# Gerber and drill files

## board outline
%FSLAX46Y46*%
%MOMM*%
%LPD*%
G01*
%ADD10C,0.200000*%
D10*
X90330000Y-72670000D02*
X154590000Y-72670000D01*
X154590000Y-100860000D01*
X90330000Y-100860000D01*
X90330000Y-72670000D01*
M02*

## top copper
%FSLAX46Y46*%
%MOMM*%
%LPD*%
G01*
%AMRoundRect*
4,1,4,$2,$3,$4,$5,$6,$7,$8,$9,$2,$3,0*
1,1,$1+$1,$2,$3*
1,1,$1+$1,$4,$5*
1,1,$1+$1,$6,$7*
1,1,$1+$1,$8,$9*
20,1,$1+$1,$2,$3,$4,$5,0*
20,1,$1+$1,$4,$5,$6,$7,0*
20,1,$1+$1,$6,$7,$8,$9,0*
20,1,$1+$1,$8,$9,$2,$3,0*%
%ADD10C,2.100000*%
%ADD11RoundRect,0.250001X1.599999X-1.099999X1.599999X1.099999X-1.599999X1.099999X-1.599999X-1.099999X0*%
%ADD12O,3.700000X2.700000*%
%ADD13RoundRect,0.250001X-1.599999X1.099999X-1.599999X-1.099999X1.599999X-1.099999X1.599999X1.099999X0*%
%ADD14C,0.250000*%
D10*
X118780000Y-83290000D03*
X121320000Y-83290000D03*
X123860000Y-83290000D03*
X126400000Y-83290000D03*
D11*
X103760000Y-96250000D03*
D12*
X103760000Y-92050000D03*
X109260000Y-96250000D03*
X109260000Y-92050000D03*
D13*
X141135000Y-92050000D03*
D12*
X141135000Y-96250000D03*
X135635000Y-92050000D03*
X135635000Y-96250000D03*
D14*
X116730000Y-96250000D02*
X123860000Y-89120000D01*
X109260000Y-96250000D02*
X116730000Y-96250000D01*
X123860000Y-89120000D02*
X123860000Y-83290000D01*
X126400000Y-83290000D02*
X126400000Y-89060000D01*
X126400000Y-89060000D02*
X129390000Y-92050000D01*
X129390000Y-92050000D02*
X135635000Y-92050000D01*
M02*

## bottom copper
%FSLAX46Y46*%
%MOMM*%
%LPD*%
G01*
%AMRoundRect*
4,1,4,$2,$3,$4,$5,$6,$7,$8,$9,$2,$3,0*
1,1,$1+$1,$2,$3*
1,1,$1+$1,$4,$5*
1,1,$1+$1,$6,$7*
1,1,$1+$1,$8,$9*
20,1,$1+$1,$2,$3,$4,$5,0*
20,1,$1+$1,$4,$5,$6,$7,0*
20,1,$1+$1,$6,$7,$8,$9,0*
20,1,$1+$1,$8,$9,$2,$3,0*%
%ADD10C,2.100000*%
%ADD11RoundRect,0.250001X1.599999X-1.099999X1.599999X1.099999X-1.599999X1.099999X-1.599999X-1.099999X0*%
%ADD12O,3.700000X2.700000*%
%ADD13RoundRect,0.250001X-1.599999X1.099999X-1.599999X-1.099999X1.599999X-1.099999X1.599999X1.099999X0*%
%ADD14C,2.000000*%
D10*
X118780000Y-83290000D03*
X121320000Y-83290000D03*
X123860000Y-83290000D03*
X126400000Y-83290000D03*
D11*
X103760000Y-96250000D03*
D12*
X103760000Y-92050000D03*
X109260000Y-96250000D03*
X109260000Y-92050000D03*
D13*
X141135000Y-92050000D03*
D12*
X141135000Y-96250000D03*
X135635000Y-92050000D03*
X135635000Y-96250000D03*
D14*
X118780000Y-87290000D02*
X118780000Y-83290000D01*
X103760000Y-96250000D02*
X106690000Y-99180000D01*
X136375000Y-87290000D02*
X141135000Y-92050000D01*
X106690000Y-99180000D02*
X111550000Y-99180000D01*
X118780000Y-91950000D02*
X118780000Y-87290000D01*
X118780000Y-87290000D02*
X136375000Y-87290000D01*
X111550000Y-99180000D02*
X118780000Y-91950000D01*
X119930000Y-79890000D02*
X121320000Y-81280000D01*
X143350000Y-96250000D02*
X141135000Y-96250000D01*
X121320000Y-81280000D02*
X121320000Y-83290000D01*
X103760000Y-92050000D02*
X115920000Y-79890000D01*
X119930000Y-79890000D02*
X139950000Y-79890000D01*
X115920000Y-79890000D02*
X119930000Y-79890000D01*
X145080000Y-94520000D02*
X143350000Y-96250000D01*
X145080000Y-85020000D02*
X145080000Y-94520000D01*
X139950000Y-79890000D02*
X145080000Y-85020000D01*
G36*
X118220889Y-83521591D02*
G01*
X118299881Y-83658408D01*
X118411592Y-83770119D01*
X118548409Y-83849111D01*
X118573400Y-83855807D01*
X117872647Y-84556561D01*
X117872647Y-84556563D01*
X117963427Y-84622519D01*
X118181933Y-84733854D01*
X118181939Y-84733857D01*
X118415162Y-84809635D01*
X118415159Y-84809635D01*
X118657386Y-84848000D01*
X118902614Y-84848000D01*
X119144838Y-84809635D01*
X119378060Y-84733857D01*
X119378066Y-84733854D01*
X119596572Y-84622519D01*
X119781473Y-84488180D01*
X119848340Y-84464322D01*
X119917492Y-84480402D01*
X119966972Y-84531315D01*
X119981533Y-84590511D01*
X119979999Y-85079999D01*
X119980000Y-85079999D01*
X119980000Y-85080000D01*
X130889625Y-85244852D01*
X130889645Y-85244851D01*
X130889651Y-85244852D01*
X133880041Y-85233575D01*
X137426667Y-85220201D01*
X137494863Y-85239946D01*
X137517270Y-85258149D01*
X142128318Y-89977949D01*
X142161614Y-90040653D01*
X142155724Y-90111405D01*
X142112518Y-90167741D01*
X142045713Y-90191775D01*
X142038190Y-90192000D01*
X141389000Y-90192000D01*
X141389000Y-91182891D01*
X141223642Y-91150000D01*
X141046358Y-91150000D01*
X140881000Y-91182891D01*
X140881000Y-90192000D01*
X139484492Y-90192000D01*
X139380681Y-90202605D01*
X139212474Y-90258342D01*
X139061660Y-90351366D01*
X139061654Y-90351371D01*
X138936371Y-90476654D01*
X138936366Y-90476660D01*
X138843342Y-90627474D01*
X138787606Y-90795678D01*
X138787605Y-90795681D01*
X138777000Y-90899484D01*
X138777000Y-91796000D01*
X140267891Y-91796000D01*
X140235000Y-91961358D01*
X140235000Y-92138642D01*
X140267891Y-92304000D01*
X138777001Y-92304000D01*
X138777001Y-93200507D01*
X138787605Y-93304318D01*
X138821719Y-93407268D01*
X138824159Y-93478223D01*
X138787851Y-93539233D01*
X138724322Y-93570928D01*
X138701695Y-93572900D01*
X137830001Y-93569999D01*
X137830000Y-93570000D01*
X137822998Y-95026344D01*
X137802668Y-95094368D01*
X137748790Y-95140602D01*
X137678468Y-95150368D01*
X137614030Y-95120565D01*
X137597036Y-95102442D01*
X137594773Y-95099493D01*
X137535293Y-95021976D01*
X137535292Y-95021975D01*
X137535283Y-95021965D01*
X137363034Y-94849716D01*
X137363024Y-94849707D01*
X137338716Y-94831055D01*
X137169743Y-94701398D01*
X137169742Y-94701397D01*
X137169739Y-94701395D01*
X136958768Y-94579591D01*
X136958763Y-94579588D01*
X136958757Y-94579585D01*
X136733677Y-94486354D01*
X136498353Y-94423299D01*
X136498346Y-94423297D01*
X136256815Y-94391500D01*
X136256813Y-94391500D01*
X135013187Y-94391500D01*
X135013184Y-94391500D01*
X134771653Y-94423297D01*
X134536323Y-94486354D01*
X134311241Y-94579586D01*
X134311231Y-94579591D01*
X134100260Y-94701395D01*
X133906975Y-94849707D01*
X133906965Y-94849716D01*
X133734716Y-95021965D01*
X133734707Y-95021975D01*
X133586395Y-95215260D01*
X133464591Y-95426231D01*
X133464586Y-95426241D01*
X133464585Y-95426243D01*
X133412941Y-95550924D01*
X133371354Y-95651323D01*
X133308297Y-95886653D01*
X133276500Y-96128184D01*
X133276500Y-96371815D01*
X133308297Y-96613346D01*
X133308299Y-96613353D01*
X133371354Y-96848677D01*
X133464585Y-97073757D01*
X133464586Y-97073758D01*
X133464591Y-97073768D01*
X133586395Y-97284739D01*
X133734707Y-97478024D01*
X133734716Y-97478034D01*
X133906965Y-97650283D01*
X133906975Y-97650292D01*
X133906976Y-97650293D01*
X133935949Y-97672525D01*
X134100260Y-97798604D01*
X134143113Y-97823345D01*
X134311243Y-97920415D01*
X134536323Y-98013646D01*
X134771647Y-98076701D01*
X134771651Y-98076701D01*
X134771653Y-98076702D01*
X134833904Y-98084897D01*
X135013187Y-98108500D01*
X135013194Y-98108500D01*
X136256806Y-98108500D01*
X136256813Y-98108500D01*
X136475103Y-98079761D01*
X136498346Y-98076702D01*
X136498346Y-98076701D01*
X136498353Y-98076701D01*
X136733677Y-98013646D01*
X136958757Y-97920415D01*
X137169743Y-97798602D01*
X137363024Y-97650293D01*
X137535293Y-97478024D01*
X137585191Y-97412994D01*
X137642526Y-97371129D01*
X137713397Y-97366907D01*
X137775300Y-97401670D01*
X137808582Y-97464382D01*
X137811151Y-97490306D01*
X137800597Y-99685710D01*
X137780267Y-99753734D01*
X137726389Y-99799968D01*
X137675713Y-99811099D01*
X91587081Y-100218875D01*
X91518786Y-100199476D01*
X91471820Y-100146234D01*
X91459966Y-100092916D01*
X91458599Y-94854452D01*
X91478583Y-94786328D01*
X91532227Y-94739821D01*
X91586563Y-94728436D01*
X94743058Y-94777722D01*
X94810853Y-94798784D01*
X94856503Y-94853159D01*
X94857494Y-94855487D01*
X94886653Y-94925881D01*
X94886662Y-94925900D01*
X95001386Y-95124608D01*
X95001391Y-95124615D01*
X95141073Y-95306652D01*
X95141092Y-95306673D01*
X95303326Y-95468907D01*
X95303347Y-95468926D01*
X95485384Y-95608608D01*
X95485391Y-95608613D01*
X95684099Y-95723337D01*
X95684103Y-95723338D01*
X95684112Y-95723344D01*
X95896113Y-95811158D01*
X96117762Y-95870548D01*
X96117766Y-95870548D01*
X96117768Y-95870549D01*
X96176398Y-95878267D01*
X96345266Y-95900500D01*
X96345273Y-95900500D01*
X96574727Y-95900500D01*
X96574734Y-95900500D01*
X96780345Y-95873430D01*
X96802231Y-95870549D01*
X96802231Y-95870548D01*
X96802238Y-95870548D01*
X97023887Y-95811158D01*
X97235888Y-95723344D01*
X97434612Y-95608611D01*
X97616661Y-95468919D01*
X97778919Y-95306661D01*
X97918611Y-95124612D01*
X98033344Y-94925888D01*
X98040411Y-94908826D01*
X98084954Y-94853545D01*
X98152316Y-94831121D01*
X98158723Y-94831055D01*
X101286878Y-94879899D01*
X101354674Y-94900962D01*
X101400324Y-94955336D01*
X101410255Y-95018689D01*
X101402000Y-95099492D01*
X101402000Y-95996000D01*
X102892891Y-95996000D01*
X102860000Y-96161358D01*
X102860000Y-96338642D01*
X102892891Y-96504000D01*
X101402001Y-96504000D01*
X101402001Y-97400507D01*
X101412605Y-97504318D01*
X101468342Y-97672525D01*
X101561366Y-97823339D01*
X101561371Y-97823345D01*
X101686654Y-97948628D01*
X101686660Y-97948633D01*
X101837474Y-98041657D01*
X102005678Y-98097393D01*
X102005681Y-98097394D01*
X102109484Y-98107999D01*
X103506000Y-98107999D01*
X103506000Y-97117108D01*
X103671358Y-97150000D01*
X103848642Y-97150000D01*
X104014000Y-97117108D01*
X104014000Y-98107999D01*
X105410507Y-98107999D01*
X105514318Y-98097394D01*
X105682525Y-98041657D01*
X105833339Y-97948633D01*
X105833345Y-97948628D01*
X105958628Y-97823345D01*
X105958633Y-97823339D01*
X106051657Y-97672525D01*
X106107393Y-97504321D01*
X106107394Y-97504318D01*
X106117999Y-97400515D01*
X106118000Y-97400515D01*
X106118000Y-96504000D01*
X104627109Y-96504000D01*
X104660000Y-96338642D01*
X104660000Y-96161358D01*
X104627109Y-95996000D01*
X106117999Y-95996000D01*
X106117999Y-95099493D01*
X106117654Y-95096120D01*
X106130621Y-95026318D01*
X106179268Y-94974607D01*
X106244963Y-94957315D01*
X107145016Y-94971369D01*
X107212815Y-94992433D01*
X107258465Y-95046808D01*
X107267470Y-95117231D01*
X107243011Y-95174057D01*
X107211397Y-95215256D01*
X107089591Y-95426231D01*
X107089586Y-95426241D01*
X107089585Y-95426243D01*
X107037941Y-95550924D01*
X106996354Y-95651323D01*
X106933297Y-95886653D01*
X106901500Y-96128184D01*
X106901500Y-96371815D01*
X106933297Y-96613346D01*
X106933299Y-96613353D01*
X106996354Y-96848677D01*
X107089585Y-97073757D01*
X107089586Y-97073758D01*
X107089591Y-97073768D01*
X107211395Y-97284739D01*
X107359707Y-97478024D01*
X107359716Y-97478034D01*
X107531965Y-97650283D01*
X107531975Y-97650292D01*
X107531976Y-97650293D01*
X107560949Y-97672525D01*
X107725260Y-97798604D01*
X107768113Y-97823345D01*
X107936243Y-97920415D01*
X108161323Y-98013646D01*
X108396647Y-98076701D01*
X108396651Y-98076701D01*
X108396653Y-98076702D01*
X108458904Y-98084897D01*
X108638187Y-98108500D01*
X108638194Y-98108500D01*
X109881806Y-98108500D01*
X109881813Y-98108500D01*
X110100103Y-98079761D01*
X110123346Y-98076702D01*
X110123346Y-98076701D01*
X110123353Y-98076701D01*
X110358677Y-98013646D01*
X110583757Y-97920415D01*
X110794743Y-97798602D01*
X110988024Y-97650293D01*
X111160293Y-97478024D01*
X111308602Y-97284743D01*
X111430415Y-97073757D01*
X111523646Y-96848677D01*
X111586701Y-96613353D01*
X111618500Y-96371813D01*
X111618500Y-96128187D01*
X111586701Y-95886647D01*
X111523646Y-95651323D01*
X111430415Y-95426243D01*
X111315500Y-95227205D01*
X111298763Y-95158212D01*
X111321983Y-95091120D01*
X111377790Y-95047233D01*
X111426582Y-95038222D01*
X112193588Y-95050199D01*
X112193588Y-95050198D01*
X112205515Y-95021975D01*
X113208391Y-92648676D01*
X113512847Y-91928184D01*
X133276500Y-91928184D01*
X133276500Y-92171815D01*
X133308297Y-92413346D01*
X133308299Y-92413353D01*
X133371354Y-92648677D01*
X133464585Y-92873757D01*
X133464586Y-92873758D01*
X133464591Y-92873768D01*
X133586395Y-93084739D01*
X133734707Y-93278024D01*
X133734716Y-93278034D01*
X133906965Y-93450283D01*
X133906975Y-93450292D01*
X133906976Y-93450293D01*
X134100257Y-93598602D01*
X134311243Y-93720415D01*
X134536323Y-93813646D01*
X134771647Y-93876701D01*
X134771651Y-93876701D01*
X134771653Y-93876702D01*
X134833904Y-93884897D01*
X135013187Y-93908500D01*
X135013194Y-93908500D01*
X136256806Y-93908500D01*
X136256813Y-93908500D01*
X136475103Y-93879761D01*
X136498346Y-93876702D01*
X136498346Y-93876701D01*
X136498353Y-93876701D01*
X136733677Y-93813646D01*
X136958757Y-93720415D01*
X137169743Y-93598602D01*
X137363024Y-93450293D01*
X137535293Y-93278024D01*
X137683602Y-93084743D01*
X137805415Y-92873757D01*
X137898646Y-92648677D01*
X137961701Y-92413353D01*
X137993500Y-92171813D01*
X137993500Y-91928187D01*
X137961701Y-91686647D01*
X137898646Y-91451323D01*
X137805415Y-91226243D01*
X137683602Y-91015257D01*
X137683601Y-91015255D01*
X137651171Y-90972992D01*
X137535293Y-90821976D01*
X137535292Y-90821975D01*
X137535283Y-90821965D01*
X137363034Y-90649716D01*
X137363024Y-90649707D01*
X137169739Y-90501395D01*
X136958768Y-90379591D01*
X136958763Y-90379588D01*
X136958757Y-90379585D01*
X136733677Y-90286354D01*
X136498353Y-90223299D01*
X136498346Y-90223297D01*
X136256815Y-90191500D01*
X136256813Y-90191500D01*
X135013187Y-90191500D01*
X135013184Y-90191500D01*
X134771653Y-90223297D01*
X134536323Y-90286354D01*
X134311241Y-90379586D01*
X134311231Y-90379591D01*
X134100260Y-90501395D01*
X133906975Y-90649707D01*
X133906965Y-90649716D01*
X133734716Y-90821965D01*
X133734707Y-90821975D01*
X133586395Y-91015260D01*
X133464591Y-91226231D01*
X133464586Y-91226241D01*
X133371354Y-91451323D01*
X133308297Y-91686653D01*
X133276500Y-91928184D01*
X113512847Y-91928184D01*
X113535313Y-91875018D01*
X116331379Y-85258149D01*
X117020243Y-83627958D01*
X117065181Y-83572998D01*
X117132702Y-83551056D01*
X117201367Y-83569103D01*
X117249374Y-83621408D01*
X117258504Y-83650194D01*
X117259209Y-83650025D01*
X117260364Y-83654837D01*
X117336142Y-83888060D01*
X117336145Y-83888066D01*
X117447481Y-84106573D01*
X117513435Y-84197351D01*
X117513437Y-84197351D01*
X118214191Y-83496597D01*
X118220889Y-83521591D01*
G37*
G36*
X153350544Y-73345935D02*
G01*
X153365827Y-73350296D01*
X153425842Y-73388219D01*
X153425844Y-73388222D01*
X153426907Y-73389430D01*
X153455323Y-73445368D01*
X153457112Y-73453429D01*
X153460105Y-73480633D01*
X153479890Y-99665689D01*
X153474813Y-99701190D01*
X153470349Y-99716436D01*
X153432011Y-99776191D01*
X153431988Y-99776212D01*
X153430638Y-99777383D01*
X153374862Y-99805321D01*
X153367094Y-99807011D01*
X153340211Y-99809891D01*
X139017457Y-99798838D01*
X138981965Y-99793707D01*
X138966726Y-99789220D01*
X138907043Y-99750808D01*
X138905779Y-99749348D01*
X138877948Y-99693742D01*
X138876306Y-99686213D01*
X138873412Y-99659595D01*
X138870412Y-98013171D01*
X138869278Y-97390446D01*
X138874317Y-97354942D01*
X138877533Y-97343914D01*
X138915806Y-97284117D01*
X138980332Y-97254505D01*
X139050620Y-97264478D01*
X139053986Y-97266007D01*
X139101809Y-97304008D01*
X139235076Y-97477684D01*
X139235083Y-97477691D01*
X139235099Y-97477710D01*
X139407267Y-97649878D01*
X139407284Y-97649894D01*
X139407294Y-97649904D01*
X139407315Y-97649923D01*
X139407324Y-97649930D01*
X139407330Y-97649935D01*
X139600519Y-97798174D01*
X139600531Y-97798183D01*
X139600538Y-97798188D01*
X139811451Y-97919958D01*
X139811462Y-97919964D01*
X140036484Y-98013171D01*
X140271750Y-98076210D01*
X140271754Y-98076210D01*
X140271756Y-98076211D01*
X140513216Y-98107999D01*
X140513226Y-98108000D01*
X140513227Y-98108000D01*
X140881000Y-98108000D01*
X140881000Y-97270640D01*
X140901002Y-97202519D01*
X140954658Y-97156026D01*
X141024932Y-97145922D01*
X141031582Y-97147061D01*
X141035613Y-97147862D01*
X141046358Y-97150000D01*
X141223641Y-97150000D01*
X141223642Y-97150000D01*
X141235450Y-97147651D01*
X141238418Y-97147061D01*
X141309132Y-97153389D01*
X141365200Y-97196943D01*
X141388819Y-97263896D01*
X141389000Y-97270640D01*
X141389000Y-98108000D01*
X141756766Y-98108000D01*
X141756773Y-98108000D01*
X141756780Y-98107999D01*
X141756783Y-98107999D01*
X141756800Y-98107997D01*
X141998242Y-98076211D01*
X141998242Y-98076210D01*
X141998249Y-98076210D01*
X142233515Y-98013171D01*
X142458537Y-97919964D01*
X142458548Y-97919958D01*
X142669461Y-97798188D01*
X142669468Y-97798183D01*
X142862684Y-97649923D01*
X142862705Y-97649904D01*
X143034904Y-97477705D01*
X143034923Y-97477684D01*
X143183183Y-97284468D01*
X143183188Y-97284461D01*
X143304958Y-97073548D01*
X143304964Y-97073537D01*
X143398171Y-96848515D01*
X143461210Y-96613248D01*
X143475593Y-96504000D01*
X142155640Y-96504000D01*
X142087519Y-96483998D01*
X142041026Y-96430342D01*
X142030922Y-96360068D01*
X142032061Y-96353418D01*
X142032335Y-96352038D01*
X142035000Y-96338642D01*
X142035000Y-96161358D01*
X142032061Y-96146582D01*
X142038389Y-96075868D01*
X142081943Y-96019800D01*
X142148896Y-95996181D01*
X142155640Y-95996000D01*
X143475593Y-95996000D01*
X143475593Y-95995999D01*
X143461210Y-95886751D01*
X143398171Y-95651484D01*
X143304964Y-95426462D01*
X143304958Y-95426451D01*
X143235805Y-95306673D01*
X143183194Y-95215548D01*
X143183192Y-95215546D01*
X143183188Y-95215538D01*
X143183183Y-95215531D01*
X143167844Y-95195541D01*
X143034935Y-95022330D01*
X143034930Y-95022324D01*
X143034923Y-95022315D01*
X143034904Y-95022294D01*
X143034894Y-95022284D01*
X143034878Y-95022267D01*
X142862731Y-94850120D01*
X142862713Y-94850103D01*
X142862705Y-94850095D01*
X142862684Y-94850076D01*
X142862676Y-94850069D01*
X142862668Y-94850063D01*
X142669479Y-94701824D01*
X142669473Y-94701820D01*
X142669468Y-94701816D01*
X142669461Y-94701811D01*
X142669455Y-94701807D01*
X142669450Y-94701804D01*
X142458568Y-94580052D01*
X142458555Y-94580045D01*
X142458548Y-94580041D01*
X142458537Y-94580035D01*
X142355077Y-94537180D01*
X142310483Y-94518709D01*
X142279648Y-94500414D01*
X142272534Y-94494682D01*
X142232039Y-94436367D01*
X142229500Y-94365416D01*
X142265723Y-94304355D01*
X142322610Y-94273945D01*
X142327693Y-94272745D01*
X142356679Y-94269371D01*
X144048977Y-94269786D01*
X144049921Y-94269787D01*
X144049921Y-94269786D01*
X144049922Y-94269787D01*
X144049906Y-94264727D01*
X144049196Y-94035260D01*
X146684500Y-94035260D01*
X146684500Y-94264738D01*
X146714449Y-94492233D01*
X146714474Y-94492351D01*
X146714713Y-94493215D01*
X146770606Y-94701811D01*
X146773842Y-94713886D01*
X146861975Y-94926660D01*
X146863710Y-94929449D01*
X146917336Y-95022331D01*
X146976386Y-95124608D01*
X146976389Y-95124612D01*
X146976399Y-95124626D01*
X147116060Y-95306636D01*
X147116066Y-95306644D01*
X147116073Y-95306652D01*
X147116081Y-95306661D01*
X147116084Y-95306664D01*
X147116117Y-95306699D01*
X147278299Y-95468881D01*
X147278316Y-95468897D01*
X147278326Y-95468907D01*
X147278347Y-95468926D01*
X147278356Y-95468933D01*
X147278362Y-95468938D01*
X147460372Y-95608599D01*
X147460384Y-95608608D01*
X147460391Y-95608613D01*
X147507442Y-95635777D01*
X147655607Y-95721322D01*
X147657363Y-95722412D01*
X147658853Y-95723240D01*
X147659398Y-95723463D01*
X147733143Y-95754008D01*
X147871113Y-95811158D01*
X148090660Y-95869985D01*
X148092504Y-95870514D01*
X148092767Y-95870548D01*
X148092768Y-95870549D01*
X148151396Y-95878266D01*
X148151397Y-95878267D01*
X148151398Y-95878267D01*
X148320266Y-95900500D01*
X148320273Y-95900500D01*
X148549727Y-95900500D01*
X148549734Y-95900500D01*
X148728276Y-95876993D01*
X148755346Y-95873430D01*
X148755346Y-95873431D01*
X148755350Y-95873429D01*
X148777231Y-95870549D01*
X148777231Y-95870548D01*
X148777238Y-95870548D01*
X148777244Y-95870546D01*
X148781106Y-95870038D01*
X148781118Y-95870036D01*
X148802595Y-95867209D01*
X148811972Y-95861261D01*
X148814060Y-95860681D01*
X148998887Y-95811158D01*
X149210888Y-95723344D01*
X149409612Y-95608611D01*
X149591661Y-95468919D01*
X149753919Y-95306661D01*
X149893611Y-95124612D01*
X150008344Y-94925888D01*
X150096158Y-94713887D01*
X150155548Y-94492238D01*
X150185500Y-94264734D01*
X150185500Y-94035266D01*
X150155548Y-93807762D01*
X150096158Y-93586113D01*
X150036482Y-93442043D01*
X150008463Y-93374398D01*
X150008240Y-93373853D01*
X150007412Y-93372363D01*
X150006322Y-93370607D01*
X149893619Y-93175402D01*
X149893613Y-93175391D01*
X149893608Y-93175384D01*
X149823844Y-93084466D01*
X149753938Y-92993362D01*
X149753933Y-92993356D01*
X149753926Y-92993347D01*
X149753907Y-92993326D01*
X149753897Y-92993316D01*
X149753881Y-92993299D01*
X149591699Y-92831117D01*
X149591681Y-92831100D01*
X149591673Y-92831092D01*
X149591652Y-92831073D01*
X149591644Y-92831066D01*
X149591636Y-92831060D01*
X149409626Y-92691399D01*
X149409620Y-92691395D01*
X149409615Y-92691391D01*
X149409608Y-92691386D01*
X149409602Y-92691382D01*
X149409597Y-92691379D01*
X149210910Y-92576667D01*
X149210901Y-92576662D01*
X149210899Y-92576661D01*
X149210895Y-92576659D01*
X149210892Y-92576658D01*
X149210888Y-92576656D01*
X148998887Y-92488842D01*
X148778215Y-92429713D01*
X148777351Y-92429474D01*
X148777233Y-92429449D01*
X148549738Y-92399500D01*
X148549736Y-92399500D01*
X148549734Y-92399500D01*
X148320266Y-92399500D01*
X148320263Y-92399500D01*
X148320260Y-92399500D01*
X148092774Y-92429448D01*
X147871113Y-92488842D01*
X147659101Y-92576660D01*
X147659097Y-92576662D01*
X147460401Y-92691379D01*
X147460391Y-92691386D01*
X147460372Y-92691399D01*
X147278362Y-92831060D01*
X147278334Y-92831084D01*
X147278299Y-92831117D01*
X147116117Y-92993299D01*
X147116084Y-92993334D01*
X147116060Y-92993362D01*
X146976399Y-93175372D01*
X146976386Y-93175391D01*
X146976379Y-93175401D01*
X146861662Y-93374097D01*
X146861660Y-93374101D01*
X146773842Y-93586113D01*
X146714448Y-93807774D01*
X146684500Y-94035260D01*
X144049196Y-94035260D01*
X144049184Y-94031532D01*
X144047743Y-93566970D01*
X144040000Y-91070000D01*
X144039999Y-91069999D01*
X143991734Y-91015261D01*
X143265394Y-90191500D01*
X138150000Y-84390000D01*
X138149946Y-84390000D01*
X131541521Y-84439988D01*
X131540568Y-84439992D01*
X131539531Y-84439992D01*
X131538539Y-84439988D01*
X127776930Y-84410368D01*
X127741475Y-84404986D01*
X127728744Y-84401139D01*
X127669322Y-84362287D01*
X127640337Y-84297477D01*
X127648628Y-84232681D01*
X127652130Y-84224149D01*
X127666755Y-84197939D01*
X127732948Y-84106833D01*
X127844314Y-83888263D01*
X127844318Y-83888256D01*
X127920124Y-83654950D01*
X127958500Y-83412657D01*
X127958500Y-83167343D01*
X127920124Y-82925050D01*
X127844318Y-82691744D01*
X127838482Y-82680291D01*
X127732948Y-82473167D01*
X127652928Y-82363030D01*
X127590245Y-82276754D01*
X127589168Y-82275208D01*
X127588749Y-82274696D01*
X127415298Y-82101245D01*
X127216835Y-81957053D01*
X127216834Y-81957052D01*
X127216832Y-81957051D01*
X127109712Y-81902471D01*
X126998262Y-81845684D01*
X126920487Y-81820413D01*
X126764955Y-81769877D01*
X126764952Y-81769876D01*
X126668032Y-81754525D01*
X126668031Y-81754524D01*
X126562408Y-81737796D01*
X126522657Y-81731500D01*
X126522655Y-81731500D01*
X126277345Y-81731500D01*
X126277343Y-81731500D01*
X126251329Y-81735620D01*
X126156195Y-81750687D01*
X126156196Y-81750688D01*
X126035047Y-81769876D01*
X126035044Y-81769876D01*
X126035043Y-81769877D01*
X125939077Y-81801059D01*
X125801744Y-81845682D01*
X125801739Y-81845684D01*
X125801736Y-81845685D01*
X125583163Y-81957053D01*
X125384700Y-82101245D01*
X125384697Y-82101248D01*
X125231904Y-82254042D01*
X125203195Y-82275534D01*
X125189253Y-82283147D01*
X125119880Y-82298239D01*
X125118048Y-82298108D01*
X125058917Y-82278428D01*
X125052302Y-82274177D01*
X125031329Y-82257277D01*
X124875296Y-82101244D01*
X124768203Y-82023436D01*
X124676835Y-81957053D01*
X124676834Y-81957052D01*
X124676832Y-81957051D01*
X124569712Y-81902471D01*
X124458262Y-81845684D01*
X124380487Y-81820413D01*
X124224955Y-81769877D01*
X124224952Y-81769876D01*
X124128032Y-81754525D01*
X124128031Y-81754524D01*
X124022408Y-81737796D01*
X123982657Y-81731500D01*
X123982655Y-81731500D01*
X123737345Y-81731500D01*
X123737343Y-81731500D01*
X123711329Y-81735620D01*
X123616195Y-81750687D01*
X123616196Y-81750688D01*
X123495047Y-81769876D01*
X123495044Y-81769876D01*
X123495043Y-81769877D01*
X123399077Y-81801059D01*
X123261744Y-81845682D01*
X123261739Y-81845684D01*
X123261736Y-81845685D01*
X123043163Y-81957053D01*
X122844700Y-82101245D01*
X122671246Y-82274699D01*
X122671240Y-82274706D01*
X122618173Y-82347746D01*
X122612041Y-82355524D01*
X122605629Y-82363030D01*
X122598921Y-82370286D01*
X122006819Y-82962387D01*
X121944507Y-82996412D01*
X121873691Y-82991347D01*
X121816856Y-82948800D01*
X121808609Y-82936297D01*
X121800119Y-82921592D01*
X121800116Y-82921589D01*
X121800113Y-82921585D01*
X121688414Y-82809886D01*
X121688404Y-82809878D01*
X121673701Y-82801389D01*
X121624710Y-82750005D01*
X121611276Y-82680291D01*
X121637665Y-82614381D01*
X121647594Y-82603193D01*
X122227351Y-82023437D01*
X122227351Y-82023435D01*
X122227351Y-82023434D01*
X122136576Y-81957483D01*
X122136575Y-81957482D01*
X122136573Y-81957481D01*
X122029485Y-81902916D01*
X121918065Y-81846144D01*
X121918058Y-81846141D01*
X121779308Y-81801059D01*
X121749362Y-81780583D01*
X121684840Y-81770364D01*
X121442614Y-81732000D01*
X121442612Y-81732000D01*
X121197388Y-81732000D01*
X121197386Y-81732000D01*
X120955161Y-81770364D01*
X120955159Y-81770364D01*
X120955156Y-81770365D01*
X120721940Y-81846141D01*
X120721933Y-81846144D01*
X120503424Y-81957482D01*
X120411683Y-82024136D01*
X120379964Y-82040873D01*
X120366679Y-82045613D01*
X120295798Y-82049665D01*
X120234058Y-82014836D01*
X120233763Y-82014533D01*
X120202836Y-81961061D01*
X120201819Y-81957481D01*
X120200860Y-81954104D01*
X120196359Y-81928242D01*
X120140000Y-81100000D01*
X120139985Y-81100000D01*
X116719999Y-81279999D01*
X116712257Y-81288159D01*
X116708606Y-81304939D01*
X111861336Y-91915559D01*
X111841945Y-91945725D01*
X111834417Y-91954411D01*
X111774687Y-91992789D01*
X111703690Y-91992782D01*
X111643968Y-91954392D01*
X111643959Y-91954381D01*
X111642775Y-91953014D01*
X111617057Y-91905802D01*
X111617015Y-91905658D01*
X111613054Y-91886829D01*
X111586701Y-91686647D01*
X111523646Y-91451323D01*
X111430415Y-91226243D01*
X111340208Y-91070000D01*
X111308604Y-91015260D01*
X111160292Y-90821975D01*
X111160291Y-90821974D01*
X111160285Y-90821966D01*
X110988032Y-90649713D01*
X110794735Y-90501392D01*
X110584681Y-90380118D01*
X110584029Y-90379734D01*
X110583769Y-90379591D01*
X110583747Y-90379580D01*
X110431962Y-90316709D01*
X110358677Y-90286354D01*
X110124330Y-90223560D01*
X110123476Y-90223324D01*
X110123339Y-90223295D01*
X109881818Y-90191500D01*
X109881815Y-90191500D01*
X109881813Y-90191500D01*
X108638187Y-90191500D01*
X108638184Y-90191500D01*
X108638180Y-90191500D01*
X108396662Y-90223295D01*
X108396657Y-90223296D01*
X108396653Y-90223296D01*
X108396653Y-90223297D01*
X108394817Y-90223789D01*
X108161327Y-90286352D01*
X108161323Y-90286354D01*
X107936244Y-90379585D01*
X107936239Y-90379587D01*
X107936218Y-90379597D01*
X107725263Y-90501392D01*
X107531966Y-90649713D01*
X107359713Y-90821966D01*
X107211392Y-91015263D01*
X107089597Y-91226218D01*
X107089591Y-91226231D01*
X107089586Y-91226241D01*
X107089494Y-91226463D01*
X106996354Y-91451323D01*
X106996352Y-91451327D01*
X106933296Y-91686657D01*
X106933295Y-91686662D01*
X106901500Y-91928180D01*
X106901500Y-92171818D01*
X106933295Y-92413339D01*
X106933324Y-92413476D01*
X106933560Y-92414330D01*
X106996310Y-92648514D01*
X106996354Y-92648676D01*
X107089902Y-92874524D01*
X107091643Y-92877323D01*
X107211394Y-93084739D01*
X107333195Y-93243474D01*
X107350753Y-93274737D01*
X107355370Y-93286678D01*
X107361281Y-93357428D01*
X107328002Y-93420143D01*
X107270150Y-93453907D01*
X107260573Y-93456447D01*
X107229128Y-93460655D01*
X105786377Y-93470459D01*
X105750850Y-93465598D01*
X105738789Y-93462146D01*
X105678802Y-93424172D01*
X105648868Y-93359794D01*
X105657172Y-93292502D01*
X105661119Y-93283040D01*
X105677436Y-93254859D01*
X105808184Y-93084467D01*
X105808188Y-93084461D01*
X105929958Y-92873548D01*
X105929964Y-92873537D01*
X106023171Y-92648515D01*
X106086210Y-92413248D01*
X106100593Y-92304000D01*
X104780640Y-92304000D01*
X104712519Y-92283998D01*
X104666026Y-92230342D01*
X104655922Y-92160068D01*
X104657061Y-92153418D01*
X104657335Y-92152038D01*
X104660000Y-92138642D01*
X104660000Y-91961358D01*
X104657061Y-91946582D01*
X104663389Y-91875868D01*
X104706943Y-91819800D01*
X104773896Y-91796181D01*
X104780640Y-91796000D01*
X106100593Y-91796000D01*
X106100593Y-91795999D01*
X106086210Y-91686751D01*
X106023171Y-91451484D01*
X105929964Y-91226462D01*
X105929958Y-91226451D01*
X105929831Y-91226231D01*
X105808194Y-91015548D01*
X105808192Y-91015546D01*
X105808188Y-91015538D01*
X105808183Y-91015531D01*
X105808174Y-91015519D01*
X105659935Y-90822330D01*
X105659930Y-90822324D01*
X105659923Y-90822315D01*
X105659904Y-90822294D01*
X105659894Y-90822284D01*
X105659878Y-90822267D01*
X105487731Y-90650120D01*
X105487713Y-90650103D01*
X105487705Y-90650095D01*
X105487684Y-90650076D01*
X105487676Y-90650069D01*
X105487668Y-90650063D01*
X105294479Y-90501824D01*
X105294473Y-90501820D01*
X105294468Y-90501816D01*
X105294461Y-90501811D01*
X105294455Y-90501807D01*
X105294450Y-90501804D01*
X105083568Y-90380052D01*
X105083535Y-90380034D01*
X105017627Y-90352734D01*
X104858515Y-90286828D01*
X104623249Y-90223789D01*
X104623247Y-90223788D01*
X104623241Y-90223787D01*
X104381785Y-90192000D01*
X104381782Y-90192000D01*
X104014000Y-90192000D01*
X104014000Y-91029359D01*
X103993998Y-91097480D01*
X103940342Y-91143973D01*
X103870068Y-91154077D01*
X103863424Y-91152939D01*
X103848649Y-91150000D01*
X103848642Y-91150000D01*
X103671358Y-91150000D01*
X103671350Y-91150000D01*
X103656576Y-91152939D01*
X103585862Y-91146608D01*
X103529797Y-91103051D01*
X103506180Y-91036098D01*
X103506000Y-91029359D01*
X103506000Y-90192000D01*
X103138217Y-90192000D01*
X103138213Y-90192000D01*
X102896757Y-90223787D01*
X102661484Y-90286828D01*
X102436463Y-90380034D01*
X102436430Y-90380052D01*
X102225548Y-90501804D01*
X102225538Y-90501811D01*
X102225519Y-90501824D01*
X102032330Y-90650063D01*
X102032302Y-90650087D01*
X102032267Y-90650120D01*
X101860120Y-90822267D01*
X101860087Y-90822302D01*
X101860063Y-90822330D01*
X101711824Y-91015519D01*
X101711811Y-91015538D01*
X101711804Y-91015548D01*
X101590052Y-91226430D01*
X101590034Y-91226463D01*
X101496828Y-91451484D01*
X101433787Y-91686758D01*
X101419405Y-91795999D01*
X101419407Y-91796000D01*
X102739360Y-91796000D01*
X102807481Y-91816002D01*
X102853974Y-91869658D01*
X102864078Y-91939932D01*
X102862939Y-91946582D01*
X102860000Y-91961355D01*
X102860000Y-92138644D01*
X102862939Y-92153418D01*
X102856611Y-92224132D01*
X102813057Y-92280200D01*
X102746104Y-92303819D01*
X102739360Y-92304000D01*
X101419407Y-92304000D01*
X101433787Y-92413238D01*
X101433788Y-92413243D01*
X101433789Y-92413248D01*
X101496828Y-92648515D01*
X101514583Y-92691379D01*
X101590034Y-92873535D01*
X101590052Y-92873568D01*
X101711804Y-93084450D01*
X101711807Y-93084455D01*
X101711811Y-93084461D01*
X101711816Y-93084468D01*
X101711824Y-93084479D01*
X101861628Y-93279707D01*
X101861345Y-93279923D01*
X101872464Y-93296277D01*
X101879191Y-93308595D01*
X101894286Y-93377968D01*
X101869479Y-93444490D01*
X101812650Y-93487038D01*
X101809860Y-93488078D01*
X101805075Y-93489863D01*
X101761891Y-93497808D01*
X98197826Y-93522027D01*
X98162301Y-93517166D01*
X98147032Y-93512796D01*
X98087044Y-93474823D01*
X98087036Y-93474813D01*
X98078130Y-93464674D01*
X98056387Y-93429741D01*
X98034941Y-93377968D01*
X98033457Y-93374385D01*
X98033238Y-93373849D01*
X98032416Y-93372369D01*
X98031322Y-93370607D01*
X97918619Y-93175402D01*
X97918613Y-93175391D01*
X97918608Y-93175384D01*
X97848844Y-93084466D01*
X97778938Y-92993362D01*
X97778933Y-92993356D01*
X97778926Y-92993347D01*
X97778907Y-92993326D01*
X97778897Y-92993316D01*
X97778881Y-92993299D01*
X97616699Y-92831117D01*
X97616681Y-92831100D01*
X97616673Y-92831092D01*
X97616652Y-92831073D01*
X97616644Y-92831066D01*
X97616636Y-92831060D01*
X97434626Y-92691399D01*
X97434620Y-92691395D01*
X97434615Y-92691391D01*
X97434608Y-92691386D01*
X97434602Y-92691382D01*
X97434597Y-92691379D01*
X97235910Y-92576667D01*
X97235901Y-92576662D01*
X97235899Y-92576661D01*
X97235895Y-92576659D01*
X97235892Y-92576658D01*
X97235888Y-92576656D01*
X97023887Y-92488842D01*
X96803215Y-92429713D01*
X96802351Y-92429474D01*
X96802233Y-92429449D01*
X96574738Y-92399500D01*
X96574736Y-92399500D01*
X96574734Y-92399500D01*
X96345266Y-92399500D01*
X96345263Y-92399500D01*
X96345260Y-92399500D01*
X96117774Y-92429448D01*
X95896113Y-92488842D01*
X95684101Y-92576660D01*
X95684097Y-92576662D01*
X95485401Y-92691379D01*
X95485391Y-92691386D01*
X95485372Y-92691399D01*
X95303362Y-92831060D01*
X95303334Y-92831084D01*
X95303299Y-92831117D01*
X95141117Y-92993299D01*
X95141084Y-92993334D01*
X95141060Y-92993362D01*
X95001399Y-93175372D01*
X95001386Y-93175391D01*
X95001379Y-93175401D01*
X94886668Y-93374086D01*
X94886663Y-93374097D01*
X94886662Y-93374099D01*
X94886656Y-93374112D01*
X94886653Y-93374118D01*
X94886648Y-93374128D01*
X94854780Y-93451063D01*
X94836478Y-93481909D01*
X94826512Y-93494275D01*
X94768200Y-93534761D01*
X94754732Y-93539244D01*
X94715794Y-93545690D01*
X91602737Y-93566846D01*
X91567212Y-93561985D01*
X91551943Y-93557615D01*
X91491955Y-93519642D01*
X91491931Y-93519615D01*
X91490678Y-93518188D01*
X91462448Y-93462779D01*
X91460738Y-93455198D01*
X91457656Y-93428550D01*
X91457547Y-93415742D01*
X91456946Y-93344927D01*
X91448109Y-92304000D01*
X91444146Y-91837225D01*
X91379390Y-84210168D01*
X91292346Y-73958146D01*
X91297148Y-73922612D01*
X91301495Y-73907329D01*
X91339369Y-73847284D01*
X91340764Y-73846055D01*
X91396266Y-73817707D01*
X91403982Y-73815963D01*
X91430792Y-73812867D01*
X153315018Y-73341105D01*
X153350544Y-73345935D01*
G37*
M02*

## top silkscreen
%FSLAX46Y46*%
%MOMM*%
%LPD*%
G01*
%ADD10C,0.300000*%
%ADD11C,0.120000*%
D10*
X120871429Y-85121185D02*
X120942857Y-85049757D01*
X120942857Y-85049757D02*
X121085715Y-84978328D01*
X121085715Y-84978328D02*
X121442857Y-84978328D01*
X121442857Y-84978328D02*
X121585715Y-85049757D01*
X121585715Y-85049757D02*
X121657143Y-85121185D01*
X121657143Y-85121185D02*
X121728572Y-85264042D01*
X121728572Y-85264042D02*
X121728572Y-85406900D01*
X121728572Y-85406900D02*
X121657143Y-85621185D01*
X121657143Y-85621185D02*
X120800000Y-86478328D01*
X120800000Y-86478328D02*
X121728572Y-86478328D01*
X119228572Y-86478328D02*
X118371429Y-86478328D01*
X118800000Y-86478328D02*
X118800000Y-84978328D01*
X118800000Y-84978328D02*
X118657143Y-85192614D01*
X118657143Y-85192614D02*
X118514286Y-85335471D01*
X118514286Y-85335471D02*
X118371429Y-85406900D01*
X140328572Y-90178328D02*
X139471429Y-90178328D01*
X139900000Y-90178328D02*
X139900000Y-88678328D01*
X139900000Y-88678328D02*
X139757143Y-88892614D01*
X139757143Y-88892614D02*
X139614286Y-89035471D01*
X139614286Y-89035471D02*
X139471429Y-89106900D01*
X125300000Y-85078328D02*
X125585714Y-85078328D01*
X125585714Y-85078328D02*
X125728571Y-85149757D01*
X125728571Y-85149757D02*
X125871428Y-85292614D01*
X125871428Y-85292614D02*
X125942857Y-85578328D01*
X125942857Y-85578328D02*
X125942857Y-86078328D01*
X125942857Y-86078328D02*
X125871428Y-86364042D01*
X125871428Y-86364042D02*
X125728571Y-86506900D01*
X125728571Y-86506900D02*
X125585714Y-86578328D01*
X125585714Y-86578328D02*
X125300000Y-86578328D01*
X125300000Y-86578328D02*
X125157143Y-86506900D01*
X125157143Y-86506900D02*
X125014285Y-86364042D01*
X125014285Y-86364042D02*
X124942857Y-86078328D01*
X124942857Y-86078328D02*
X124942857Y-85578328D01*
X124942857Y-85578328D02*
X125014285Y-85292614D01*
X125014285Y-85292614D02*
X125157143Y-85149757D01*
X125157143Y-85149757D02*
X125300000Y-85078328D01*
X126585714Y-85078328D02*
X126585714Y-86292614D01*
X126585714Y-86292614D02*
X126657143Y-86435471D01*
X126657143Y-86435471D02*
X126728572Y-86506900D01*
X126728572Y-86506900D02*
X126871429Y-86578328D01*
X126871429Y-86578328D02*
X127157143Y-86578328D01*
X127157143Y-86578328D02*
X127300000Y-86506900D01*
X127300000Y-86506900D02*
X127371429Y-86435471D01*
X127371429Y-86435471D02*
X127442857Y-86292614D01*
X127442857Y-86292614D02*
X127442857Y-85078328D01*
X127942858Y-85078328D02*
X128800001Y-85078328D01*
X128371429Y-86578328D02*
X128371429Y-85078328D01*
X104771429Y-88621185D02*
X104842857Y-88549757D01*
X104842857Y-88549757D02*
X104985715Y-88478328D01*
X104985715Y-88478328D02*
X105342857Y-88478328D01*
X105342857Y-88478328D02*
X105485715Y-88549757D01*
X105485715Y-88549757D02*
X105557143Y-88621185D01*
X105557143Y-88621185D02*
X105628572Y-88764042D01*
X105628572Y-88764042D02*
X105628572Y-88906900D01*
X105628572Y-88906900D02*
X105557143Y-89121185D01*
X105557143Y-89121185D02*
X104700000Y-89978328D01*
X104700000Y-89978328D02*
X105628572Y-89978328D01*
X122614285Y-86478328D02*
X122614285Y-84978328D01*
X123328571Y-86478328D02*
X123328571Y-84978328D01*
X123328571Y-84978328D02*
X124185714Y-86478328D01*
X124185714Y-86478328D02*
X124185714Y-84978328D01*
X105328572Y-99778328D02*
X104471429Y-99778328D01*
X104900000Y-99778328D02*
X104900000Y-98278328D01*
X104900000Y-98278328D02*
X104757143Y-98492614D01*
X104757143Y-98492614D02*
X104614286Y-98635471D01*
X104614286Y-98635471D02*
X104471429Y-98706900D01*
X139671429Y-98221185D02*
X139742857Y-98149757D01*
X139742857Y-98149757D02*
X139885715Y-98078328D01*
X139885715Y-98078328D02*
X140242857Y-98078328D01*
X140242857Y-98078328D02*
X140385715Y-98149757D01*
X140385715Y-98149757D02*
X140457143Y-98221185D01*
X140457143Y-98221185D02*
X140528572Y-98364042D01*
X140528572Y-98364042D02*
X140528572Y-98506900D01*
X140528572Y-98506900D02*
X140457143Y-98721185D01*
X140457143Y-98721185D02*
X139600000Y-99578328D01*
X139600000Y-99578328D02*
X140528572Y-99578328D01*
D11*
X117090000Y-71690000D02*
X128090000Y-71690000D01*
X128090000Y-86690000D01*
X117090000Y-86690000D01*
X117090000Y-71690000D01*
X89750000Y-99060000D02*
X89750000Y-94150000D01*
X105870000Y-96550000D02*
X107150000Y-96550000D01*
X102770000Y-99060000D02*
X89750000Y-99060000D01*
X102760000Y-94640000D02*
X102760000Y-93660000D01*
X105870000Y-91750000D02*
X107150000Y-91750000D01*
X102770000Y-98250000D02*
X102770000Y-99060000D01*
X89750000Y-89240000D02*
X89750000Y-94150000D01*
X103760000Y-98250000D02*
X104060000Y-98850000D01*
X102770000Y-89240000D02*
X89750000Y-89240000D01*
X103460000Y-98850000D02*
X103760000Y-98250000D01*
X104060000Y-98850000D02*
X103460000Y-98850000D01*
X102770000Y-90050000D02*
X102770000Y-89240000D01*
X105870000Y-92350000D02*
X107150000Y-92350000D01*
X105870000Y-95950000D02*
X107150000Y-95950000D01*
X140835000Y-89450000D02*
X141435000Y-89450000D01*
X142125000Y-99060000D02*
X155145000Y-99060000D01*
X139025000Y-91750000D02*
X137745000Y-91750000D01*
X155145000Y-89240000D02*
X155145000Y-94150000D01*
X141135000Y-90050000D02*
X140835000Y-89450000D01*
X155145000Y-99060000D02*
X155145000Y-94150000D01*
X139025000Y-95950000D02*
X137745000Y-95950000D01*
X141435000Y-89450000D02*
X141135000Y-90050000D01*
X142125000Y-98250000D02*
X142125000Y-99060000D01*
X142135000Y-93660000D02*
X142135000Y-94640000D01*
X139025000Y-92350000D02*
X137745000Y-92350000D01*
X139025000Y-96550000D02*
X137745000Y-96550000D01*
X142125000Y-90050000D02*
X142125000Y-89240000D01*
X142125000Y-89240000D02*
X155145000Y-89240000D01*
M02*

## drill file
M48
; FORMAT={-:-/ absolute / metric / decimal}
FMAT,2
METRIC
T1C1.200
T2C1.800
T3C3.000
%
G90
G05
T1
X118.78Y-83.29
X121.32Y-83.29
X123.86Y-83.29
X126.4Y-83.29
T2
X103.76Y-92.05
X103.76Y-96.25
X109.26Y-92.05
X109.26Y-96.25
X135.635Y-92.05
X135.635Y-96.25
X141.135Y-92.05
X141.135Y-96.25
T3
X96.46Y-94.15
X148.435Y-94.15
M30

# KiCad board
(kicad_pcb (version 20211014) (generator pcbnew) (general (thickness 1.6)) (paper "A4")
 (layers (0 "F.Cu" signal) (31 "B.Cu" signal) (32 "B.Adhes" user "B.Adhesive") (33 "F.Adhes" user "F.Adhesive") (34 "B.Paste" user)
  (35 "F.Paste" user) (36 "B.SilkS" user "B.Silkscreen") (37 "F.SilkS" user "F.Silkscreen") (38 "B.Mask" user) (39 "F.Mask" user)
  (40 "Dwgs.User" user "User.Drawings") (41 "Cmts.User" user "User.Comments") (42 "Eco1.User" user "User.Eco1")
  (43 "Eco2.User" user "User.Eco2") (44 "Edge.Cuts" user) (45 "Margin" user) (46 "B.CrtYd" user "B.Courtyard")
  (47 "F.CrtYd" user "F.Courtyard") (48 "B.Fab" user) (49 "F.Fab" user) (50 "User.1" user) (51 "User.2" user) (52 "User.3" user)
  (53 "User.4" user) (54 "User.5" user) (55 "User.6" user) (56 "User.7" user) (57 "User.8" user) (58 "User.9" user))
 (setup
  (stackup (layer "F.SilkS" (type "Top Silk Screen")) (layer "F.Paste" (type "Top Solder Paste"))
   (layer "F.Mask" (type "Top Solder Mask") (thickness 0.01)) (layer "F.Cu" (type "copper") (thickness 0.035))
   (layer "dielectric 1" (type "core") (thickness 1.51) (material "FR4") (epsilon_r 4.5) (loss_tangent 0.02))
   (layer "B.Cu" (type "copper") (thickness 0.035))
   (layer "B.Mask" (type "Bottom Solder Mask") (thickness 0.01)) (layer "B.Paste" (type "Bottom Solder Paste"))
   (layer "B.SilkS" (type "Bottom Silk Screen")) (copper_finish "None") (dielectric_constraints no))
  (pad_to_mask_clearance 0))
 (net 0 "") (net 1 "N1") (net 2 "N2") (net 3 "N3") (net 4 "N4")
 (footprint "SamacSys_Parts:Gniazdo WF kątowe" (layer "F.Cu") (at 118.79 83.29)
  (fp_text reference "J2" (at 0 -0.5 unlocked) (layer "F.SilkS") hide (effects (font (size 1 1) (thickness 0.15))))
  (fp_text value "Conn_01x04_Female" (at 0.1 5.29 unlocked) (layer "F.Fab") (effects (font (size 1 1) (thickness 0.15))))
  (fp_rect (start -1.7 3.4) (end 9.3 -11.6) (layer "F.SilkS") (width 0.12) (fill none))
  (pad "1" thru_hole circle (at -0.01 0) (size 2.1 2.1) (drill 1.2) (layers *.Cu *.Mask) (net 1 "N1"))
  (pad "2" thru_hole circle (at 2.53 0) (size 2.1 2.1) (drill 1.2) (layers *.Cu *.Mask) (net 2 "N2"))
  (pad "3" thru_hole circle (at 5.07 0) (size 2.1 2.1) (drill 1.2) (layers *.Cu *.Mask) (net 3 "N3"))
  (pad "4" thru_hole circle (at 7.61 0) (size 2.1 2.1) (drill 1.2) (layers *.Cu *.Mask) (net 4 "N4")))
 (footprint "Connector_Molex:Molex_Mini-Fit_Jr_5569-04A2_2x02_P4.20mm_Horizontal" (layer "F.Cu") (at 103.76 96.25 90)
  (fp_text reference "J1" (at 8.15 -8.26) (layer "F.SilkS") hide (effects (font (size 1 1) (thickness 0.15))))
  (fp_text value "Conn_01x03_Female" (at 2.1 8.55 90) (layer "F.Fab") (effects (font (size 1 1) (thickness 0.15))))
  (fp_line (start -2.81 -14.01) (end 2.1 -14.01) (layer "F.SilkS") (width 0.12))
  (fp_line (start -0.3 2.11) (end -0.3 3.39) (layer "F.SilkS") (width 0.12))
  (fp_line (start -2.81 -0.99) (end -2.81 -14.01) (layer "F.SilkS") (width 0.12))
  (fp_line (start 1.61 -1) (end 2.59 -1) (layer "F.SilkS") (width 0.12))
  (fp_line (start 4.5 2.11) (end 4.5 3.39) (layer "F.SilkS") (width 0.12))
  (fp_line (start -2 -0.99) (end -2.81 -0.99) (layer "F.SilkS") (width 0.12))
  (fp_line (start 7.01 -14.01) (end 2.1 -14.01) (layer "F.SilkS") (width 0.12))
  (fp_line (start -2 0) (end -2.6 0.3) (layer "F.SilkS") (width 0.12))
  (fp_line (start 7.01 -0.99) (end 7.01 -14.01) (layer "F.SilkS") (width 0.12))
  (fp_line (start -2.6 -0.3) (end -2 0) (layer "F.SilkS") (width 0.12))
  (fp_line (start -2.6 0.3) (end -2.6 -0.3) (layer "F.SilkS") (width 0.12))
  (fp_line (start 6.2 -0.99) (end 7.01 -0.99) (layer "F.SilkS") (width 0.12))
  (fp_line (start 3.9 2.11) (end 3.9 3.39) (layer "F.SilkS") (width 0.12))
  (fp_line (start 0.3 2.11) (end 0.3 3.39) (layer "F.SilkS") (width 0.12))
  (pad "" np_thru_hole circle (at 2.1 -7.3 90) (size 3 3) (drill 3) (layers *.Cu *.Mask))
  (pad "1" thru_hole roundrect (at 0 0 90) (size 2.7 3.7) (drill 1.8) (layers *.Cu *.Mask) (roundrect_rratio 0.09259296296) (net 1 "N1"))
  (pad "2" thru_hole oval (at 4.2 0 90) (size 2.7 3.7) (drill 1.8) (layers *.Cu *.Mask) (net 2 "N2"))
  (pad "3" thru_hole oval (at 0 5.5 90) (size 2.7 3.7) (drill 1.8) (layers *.Cu *.Mask) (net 3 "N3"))
  (pad "4" thru_hole oval (at 4.2 5.5 90) (size 2.7 3.7) (drill 1.8) (layers *.Cu *.Mask)))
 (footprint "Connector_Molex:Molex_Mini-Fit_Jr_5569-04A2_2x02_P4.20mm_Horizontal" (layer "F.Cu") (at 141.135 92.05 -90)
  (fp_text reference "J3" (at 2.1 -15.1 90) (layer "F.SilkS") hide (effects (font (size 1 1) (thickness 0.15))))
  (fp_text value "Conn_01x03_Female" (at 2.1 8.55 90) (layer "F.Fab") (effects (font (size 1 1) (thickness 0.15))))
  (fp_line (start -2.6 0.3) (end -2.6 -0.3) (layer "F.SilkS") (width 0.12))
  (fp_line (start 7.01 -0.99) (end 7.01 -14.01) (layer "F.SilkS") (width 0.12))
  (fp_line (start -0.3 2.11) (end -0.3 3.39) (layer "F.SilkS") (width 0.12))
  (fp_line (start -2.81 -14.01) (end 2.1 -14.01) (layer "F.SilkS") (width 0.12))
  (fp_line (start -2 0) (end -2.6 0.3) (layer "F.SilkS") (width 0.12))
  (fp_line (start 7.01 -14.01) (end 2.1 -14.01) (layer "F.SilkS") (width 0.12))
  (fp_line (start 3.9 2.11) (end 3.9 3.39) (layer "F.SilkS") (width 0.12))
  (fp_line (start -2.6 -0.3) (end -2 0) (layer "F.SilkS") (width 0.12))
  (fp_line (start 6.2 -0.99) (end 7.01 -0.99) (layer "F.SilkS") (width 0.12))
  (fp_line (start 1.61 -1) (end 2.59 -1) (layer "F.SilkS") (width 0.12))
  (fp_line (start 0.3 2.11) (end 0.3 3.39) (layer "F.SilkS") (width 0.12))
  (fp_line (start 4.5 2.11) (end 4.5 3.39) (layer "F.SilkS") (width 0.12))
  (fp_line (start -2 -0.99) (end -2.81 -0.99) (layer "F.SilkS") (width 0.12))
  (fp_line (start -2.81 -0.99) (end -2.81 -14.01) (layer "F.SilkS") (width 0.12))
  (pad "" np_thru_hole circle (at 2.1 -7.3 270) (size 3 3) (drill 3) (layers *.Cu *.Mask))
  (pad "1" thru_hole roundrect (at 0 0 270) (size 2.7 3.7) (drill 1.8) (layers *.Cu *.Mask) (roundrect_rratio 0.09259296296) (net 1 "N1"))
  (pad "2" thru_hole oval (at 4.2 0 270) (size 2.7 3.7) (drill 1.8) (layers *.Cu *.Mask) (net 2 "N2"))
  (pad "3" thru_hole oval (at 0 5.5 270) (size 2.7 3.7) (drill 1.8) (layers *.Cu *.Mask) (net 4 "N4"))
  (pad "4" thru_hole oval (at 4.2 5.5 270) (size 2.7 3.7) (drill 1.8) (layers *.Cu *.Mask)))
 (gr_rect (start 90.33 72.67) (end 154.59 100.86) (layer "Edge.Cuts") (width 0.2) (fill none))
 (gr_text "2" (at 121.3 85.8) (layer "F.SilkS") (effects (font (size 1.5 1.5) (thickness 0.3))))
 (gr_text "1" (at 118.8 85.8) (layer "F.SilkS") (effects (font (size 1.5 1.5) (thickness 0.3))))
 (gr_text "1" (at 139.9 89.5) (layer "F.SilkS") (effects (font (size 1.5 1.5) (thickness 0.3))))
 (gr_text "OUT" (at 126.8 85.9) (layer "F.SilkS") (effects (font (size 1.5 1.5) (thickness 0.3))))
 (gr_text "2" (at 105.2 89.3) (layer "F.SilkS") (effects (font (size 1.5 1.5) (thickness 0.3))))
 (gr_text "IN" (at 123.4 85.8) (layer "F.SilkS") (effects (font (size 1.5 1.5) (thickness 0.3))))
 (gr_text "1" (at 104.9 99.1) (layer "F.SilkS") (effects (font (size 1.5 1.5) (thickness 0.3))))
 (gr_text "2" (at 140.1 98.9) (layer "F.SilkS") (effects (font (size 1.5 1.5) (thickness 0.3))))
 (segment (start 118.78 87.29) (end 118.78 83.29) (width 2) (layer "B.Cu") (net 1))
 (segment (start 103.76 96.25) (end 106.69 99.18) (width 2) (layer "B.Cu") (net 1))
 (segment (start 136.375 87.29) (end 141.135 92.05) (width 2) (layer "B.Cu") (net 1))
 (segment (start 106.69 99.18) (end 111.55 99.18) (width 2) (layer "B.Cu") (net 1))
 (segment (start 118.78 91.95) (end 118.78 87.29) (width 2) (layer "B.Cu") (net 1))
 (segment (start 118.78 87.29) (end 136.375 87.29) (width 2) (layer "B.Cu") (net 1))
 (segment (start 111.55 99.18) (end 118.78 91.95) (width 2) (layer "B.Cu") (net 1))
 (segment (start 119.93 79.89) (end 121.32 81.28) (width 2) (layer "B.Cu") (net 2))
 (segment (start 143.35 96.25) (end 141.135 96.25) (width 2) (layer "B.Cu") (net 2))
 (segment (start 121.32 81.28) (end 121.32 83.29) (width 2) (layer "B.Cu") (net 2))
 (segment (start 103.76 92.05) (end 115.92 79.89) (width 2) (layer "B.Cu") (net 2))
 (segment (start 119.93 79.89) (end 139.95 79.89) (width 2) (layer "B.Cu") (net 2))
 (segment (start 115.92 79.89) (end 119.93 79.89) (width 2) (layer "B.Cu") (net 2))
 (segment (start 145.08 94.52) (end 143.35 96.25) (width 2) (layer "B.Cu") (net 2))
 (segment (start 145.08 85.02) (end 145.08 94.52) (width 2) (layer "B.Cu") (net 2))
 (segment (start 139.95 79.89) (end 145.08 85.02) (width 2) (layer "B.Cu") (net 2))
 (segment (start 116.73 96.25) (end 123.86 89.12) (width 0.25) (layer "F.Cu") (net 3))
 (segment (start 109.26 96.25) (end 116.73 96.25) (width 0.25) (layer "F.Cu") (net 3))
 (segment (start 123.86 89.12) (end 123.86 83.29) (width 0.25) (layer "F.Cu") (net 3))
 (segment (start 126.4 83.29) (end 126.4 89.06) (width 0.25) (layer "F.Cu") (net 4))
 (segment (start 126.4 89.06) (end 129.39 92.05) (width 0.25) (layer "F.Cu") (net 4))
 (segment (start 129.39 92.05) (end 135.635 92.05) (width 0.25) (layer "F.Cu") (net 4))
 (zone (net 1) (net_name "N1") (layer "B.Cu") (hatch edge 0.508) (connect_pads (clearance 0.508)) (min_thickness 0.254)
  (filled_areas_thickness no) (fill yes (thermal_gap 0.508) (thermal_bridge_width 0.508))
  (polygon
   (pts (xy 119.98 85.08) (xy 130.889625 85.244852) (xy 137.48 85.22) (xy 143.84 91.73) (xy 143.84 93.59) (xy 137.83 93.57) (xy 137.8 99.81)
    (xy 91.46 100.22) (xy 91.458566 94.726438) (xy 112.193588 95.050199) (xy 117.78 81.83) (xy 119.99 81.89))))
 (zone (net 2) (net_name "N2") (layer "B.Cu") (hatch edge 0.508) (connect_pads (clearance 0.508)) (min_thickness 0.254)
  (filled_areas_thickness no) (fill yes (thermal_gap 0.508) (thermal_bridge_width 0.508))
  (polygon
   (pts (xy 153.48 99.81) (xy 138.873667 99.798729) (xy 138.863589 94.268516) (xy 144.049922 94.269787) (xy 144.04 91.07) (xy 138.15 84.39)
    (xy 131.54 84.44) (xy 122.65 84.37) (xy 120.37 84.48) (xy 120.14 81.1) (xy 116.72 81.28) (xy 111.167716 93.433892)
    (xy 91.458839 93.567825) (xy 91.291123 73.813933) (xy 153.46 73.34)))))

